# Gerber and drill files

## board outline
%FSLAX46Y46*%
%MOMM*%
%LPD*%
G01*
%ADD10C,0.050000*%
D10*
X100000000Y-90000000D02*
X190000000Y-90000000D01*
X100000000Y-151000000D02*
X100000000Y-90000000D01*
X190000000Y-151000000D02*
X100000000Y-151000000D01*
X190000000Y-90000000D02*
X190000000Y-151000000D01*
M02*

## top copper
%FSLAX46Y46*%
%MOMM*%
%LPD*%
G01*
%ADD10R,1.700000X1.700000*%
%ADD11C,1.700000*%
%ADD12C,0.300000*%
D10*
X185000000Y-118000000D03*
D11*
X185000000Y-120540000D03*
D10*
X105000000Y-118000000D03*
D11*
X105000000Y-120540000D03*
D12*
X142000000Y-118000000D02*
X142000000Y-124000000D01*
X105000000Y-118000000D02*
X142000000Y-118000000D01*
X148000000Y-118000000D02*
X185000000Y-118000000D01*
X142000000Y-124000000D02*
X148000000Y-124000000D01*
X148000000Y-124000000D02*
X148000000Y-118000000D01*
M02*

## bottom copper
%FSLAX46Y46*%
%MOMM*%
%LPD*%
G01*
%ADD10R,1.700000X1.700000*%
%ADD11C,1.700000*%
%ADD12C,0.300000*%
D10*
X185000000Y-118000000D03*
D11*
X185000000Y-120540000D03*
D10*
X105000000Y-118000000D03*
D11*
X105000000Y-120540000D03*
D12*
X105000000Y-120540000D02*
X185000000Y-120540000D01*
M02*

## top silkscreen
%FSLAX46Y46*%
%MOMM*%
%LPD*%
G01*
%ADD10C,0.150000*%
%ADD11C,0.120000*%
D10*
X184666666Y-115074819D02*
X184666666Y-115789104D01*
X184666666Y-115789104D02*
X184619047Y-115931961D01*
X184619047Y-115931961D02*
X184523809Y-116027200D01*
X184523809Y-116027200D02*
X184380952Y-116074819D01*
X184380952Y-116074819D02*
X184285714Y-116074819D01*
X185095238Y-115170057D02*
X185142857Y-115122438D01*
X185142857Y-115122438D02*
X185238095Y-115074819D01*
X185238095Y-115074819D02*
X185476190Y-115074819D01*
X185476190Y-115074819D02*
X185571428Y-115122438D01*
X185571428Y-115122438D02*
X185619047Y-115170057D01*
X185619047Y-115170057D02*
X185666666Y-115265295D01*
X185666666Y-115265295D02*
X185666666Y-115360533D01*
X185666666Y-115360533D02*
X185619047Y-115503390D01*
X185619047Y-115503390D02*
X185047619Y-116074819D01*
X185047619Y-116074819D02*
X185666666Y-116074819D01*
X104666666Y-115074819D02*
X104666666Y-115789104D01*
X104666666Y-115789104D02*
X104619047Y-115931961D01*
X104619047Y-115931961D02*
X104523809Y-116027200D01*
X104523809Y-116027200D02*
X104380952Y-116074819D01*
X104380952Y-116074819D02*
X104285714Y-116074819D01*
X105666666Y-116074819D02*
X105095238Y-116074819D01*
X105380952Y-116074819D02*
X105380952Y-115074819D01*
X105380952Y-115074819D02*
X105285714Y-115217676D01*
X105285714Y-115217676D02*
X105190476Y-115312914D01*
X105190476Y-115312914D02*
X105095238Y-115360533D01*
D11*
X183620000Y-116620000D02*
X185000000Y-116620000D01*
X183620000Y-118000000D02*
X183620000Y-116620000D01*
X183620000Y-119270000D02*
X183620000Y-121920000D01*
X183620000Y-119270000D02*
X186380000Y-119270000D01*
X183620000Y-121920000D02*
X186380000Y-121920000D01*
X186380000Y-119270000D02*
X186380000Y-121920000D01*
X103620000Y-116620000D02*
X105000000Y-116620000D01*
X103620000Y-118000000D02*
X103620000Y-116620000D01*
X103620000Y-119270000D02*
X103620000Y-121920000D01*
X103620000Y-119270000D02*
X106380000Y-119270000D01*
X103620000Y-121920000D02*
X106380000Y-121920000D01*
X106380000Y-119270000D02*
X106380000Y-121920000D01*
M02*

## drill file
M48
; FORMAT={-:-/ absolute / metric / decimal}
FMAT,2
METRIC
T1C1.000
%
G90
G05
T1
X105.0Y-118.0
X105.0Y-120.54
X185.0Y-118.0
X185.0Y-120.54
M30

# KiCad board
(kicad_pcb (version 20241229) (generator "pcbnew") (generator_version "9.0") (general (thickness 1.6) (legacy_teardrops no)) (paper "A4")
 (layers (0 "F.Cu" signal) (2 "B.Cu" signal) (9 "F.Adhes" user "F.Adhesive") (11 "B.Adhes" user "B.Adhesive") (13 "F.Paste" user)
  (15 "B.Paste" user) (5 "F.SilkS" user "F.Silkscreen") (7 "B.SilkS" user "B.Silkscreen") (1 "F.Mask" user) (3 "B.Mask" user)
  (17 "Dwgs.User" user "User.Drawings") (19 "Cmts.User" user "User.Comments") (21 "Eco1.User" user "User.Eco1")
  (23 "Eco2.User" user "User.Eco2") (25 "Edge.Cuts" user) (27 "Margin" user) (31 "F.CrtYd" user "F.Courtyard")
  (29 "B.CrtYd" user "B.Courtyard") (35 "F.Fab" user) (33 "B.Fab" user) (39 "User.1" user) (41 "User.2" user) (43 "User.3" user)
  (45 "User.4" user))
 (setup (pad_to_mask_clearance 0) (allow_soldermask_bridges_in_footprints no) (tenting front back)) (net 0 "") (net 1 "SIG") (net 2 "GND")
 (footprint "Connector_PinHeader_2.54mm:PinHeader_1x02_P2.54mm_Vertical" (layer "F.Cu") (at 185 118)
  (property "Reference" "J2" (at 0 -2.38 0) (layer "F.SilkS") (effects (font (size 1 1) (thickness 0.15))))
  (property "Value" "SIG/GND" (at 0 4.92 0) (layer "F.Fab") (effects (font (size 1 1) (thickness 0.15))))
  (fp_line (start -1.38 -1.38) (end 0 -1.38) (stroke (width 0.12) (type solid)) (layer "F.SilkS"))
  (fp_line (start -1.38 0) (end -1.38 -1.38) (stroke (width 0.12) (type solid)) (layer "F.SilkS"))
  (fp_line (start -1.38 1.27) (end -1.38 3.92) (stroke (width 0.12) (type solid)) (layer "F.SilkS"))
  (fp_line (start -1.38 1.27) (end 1.38 1.27) (stroke (width 0.12) (type solid)) (layer "F.SilkS"))
  (fp_line (start -1.38 3.92) (end 1.38 3.92) (stroke (width 0.12) (type solid)) (layer "F.SilkS"))
  (fp_line (start 1.38 1.27) (end 1.38 3.92) (stroke (width 0.12) (type solid)) (layer "F.SilkS"))
  (pad "1" thru_hole rect (at 0 0) (size 1.7 1.7) (drill 1) (layers "*.Cu" "*.Mask") (remove_unused_layers no) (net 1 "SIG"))
  (pad "2" thru_hole circle (at 0 2.54) (size 1.7 1.7) (drill 1) (layers "*.Cu" "*.Mask") (remove_unused_layers no) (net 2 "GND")))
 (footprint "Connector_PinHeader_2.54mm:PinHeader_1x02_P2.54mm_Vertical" (layer "F.Cu") (at 105 118)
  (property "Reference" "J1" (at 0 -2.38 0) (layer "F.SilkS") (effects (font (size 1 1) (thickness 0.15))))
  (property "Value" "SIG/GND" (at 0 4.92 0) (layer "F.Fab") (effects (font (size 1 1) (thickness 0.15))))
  (fp_line (start -1.38 -1.38) (end 0 -1.38) (stroke (width 0.12) (type solid)) (layer "F.SilkS"))
  (fp_line (start -1.38 0) (end -1.38 -1.38) (stroke (width 0.12) (type solid)) (layer "F.SilkS"))
  (fp_line (start -1.38 1.27) (end -1.38 3.92) (stroke (width 0.12) (type solid)) (layer "F.SilkS"))
  (fp_line (start -1.38 1.27) (end 1.38 1.27) (stroke (width 0.12) (type solid)) (layer "F.SilkS"))
  (fp_line (start -1.38 3.92) (end 1.38 3.92) (stroke (width 0.12) (type solid)) (layer "F.SilkS"))
  (fp_line (start 1.38 1.27) (end 1.38 3.92) (stroke (width 0.12) (type solid)) (layer "F.SilkS"))
  (pad "1" thru_hole rect (at 0 0) (size 1.7 1.7) (drill 1) (layers "*.Cu" "*.Mask") (remove_unused_layers no) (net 1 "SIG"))
  (pad "2" thru_hole circle (at 0 2.54) (size 1.7 1.7) (drill 1) (layers "*.Cu" "*.Mask") (remove_unused_layers no) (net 2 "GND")))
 (gr_line (start 100 90) (end 190 90) (stroke (width 0.05) (type default)) (layer "Edge.Cuts"))
 (gr_line (start 100 151) (end 100 90) (stroke (width 0.05) (type default)) (layer "Edge.Cuts"))
 (gr_line (start 190 151) (end 100 151) (stroke (width 0.05) (type default)) (layer "Edge.Cuts"))
 (gr_line (start 190 90) (end 190 151) (stroke (width 0.05) (type default)) (layer "Edge.Cuts"))
 (segment (start 142 118) (end 142 124) (width 0.3) (layer "F.Cu") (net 1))
 (segment (start 105 118) (end 142 118) (width 0.3) (layer "F.Cu") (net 1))
 (segment (start 148 118) (end 185 118) (width 0.3) (layer "F.Cu") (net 1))
 (segment (start 142 124) (end 148 124) (width 0.3) (layer "F.Cu") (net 1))
 (segment (start 148 124) (end 148 118) (width 0.3) (layer "F.Cu") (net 1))
 (segment (start 105 120.54) (end 185 120.54) (width 0.3) (layer "B.Cu") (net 2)))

